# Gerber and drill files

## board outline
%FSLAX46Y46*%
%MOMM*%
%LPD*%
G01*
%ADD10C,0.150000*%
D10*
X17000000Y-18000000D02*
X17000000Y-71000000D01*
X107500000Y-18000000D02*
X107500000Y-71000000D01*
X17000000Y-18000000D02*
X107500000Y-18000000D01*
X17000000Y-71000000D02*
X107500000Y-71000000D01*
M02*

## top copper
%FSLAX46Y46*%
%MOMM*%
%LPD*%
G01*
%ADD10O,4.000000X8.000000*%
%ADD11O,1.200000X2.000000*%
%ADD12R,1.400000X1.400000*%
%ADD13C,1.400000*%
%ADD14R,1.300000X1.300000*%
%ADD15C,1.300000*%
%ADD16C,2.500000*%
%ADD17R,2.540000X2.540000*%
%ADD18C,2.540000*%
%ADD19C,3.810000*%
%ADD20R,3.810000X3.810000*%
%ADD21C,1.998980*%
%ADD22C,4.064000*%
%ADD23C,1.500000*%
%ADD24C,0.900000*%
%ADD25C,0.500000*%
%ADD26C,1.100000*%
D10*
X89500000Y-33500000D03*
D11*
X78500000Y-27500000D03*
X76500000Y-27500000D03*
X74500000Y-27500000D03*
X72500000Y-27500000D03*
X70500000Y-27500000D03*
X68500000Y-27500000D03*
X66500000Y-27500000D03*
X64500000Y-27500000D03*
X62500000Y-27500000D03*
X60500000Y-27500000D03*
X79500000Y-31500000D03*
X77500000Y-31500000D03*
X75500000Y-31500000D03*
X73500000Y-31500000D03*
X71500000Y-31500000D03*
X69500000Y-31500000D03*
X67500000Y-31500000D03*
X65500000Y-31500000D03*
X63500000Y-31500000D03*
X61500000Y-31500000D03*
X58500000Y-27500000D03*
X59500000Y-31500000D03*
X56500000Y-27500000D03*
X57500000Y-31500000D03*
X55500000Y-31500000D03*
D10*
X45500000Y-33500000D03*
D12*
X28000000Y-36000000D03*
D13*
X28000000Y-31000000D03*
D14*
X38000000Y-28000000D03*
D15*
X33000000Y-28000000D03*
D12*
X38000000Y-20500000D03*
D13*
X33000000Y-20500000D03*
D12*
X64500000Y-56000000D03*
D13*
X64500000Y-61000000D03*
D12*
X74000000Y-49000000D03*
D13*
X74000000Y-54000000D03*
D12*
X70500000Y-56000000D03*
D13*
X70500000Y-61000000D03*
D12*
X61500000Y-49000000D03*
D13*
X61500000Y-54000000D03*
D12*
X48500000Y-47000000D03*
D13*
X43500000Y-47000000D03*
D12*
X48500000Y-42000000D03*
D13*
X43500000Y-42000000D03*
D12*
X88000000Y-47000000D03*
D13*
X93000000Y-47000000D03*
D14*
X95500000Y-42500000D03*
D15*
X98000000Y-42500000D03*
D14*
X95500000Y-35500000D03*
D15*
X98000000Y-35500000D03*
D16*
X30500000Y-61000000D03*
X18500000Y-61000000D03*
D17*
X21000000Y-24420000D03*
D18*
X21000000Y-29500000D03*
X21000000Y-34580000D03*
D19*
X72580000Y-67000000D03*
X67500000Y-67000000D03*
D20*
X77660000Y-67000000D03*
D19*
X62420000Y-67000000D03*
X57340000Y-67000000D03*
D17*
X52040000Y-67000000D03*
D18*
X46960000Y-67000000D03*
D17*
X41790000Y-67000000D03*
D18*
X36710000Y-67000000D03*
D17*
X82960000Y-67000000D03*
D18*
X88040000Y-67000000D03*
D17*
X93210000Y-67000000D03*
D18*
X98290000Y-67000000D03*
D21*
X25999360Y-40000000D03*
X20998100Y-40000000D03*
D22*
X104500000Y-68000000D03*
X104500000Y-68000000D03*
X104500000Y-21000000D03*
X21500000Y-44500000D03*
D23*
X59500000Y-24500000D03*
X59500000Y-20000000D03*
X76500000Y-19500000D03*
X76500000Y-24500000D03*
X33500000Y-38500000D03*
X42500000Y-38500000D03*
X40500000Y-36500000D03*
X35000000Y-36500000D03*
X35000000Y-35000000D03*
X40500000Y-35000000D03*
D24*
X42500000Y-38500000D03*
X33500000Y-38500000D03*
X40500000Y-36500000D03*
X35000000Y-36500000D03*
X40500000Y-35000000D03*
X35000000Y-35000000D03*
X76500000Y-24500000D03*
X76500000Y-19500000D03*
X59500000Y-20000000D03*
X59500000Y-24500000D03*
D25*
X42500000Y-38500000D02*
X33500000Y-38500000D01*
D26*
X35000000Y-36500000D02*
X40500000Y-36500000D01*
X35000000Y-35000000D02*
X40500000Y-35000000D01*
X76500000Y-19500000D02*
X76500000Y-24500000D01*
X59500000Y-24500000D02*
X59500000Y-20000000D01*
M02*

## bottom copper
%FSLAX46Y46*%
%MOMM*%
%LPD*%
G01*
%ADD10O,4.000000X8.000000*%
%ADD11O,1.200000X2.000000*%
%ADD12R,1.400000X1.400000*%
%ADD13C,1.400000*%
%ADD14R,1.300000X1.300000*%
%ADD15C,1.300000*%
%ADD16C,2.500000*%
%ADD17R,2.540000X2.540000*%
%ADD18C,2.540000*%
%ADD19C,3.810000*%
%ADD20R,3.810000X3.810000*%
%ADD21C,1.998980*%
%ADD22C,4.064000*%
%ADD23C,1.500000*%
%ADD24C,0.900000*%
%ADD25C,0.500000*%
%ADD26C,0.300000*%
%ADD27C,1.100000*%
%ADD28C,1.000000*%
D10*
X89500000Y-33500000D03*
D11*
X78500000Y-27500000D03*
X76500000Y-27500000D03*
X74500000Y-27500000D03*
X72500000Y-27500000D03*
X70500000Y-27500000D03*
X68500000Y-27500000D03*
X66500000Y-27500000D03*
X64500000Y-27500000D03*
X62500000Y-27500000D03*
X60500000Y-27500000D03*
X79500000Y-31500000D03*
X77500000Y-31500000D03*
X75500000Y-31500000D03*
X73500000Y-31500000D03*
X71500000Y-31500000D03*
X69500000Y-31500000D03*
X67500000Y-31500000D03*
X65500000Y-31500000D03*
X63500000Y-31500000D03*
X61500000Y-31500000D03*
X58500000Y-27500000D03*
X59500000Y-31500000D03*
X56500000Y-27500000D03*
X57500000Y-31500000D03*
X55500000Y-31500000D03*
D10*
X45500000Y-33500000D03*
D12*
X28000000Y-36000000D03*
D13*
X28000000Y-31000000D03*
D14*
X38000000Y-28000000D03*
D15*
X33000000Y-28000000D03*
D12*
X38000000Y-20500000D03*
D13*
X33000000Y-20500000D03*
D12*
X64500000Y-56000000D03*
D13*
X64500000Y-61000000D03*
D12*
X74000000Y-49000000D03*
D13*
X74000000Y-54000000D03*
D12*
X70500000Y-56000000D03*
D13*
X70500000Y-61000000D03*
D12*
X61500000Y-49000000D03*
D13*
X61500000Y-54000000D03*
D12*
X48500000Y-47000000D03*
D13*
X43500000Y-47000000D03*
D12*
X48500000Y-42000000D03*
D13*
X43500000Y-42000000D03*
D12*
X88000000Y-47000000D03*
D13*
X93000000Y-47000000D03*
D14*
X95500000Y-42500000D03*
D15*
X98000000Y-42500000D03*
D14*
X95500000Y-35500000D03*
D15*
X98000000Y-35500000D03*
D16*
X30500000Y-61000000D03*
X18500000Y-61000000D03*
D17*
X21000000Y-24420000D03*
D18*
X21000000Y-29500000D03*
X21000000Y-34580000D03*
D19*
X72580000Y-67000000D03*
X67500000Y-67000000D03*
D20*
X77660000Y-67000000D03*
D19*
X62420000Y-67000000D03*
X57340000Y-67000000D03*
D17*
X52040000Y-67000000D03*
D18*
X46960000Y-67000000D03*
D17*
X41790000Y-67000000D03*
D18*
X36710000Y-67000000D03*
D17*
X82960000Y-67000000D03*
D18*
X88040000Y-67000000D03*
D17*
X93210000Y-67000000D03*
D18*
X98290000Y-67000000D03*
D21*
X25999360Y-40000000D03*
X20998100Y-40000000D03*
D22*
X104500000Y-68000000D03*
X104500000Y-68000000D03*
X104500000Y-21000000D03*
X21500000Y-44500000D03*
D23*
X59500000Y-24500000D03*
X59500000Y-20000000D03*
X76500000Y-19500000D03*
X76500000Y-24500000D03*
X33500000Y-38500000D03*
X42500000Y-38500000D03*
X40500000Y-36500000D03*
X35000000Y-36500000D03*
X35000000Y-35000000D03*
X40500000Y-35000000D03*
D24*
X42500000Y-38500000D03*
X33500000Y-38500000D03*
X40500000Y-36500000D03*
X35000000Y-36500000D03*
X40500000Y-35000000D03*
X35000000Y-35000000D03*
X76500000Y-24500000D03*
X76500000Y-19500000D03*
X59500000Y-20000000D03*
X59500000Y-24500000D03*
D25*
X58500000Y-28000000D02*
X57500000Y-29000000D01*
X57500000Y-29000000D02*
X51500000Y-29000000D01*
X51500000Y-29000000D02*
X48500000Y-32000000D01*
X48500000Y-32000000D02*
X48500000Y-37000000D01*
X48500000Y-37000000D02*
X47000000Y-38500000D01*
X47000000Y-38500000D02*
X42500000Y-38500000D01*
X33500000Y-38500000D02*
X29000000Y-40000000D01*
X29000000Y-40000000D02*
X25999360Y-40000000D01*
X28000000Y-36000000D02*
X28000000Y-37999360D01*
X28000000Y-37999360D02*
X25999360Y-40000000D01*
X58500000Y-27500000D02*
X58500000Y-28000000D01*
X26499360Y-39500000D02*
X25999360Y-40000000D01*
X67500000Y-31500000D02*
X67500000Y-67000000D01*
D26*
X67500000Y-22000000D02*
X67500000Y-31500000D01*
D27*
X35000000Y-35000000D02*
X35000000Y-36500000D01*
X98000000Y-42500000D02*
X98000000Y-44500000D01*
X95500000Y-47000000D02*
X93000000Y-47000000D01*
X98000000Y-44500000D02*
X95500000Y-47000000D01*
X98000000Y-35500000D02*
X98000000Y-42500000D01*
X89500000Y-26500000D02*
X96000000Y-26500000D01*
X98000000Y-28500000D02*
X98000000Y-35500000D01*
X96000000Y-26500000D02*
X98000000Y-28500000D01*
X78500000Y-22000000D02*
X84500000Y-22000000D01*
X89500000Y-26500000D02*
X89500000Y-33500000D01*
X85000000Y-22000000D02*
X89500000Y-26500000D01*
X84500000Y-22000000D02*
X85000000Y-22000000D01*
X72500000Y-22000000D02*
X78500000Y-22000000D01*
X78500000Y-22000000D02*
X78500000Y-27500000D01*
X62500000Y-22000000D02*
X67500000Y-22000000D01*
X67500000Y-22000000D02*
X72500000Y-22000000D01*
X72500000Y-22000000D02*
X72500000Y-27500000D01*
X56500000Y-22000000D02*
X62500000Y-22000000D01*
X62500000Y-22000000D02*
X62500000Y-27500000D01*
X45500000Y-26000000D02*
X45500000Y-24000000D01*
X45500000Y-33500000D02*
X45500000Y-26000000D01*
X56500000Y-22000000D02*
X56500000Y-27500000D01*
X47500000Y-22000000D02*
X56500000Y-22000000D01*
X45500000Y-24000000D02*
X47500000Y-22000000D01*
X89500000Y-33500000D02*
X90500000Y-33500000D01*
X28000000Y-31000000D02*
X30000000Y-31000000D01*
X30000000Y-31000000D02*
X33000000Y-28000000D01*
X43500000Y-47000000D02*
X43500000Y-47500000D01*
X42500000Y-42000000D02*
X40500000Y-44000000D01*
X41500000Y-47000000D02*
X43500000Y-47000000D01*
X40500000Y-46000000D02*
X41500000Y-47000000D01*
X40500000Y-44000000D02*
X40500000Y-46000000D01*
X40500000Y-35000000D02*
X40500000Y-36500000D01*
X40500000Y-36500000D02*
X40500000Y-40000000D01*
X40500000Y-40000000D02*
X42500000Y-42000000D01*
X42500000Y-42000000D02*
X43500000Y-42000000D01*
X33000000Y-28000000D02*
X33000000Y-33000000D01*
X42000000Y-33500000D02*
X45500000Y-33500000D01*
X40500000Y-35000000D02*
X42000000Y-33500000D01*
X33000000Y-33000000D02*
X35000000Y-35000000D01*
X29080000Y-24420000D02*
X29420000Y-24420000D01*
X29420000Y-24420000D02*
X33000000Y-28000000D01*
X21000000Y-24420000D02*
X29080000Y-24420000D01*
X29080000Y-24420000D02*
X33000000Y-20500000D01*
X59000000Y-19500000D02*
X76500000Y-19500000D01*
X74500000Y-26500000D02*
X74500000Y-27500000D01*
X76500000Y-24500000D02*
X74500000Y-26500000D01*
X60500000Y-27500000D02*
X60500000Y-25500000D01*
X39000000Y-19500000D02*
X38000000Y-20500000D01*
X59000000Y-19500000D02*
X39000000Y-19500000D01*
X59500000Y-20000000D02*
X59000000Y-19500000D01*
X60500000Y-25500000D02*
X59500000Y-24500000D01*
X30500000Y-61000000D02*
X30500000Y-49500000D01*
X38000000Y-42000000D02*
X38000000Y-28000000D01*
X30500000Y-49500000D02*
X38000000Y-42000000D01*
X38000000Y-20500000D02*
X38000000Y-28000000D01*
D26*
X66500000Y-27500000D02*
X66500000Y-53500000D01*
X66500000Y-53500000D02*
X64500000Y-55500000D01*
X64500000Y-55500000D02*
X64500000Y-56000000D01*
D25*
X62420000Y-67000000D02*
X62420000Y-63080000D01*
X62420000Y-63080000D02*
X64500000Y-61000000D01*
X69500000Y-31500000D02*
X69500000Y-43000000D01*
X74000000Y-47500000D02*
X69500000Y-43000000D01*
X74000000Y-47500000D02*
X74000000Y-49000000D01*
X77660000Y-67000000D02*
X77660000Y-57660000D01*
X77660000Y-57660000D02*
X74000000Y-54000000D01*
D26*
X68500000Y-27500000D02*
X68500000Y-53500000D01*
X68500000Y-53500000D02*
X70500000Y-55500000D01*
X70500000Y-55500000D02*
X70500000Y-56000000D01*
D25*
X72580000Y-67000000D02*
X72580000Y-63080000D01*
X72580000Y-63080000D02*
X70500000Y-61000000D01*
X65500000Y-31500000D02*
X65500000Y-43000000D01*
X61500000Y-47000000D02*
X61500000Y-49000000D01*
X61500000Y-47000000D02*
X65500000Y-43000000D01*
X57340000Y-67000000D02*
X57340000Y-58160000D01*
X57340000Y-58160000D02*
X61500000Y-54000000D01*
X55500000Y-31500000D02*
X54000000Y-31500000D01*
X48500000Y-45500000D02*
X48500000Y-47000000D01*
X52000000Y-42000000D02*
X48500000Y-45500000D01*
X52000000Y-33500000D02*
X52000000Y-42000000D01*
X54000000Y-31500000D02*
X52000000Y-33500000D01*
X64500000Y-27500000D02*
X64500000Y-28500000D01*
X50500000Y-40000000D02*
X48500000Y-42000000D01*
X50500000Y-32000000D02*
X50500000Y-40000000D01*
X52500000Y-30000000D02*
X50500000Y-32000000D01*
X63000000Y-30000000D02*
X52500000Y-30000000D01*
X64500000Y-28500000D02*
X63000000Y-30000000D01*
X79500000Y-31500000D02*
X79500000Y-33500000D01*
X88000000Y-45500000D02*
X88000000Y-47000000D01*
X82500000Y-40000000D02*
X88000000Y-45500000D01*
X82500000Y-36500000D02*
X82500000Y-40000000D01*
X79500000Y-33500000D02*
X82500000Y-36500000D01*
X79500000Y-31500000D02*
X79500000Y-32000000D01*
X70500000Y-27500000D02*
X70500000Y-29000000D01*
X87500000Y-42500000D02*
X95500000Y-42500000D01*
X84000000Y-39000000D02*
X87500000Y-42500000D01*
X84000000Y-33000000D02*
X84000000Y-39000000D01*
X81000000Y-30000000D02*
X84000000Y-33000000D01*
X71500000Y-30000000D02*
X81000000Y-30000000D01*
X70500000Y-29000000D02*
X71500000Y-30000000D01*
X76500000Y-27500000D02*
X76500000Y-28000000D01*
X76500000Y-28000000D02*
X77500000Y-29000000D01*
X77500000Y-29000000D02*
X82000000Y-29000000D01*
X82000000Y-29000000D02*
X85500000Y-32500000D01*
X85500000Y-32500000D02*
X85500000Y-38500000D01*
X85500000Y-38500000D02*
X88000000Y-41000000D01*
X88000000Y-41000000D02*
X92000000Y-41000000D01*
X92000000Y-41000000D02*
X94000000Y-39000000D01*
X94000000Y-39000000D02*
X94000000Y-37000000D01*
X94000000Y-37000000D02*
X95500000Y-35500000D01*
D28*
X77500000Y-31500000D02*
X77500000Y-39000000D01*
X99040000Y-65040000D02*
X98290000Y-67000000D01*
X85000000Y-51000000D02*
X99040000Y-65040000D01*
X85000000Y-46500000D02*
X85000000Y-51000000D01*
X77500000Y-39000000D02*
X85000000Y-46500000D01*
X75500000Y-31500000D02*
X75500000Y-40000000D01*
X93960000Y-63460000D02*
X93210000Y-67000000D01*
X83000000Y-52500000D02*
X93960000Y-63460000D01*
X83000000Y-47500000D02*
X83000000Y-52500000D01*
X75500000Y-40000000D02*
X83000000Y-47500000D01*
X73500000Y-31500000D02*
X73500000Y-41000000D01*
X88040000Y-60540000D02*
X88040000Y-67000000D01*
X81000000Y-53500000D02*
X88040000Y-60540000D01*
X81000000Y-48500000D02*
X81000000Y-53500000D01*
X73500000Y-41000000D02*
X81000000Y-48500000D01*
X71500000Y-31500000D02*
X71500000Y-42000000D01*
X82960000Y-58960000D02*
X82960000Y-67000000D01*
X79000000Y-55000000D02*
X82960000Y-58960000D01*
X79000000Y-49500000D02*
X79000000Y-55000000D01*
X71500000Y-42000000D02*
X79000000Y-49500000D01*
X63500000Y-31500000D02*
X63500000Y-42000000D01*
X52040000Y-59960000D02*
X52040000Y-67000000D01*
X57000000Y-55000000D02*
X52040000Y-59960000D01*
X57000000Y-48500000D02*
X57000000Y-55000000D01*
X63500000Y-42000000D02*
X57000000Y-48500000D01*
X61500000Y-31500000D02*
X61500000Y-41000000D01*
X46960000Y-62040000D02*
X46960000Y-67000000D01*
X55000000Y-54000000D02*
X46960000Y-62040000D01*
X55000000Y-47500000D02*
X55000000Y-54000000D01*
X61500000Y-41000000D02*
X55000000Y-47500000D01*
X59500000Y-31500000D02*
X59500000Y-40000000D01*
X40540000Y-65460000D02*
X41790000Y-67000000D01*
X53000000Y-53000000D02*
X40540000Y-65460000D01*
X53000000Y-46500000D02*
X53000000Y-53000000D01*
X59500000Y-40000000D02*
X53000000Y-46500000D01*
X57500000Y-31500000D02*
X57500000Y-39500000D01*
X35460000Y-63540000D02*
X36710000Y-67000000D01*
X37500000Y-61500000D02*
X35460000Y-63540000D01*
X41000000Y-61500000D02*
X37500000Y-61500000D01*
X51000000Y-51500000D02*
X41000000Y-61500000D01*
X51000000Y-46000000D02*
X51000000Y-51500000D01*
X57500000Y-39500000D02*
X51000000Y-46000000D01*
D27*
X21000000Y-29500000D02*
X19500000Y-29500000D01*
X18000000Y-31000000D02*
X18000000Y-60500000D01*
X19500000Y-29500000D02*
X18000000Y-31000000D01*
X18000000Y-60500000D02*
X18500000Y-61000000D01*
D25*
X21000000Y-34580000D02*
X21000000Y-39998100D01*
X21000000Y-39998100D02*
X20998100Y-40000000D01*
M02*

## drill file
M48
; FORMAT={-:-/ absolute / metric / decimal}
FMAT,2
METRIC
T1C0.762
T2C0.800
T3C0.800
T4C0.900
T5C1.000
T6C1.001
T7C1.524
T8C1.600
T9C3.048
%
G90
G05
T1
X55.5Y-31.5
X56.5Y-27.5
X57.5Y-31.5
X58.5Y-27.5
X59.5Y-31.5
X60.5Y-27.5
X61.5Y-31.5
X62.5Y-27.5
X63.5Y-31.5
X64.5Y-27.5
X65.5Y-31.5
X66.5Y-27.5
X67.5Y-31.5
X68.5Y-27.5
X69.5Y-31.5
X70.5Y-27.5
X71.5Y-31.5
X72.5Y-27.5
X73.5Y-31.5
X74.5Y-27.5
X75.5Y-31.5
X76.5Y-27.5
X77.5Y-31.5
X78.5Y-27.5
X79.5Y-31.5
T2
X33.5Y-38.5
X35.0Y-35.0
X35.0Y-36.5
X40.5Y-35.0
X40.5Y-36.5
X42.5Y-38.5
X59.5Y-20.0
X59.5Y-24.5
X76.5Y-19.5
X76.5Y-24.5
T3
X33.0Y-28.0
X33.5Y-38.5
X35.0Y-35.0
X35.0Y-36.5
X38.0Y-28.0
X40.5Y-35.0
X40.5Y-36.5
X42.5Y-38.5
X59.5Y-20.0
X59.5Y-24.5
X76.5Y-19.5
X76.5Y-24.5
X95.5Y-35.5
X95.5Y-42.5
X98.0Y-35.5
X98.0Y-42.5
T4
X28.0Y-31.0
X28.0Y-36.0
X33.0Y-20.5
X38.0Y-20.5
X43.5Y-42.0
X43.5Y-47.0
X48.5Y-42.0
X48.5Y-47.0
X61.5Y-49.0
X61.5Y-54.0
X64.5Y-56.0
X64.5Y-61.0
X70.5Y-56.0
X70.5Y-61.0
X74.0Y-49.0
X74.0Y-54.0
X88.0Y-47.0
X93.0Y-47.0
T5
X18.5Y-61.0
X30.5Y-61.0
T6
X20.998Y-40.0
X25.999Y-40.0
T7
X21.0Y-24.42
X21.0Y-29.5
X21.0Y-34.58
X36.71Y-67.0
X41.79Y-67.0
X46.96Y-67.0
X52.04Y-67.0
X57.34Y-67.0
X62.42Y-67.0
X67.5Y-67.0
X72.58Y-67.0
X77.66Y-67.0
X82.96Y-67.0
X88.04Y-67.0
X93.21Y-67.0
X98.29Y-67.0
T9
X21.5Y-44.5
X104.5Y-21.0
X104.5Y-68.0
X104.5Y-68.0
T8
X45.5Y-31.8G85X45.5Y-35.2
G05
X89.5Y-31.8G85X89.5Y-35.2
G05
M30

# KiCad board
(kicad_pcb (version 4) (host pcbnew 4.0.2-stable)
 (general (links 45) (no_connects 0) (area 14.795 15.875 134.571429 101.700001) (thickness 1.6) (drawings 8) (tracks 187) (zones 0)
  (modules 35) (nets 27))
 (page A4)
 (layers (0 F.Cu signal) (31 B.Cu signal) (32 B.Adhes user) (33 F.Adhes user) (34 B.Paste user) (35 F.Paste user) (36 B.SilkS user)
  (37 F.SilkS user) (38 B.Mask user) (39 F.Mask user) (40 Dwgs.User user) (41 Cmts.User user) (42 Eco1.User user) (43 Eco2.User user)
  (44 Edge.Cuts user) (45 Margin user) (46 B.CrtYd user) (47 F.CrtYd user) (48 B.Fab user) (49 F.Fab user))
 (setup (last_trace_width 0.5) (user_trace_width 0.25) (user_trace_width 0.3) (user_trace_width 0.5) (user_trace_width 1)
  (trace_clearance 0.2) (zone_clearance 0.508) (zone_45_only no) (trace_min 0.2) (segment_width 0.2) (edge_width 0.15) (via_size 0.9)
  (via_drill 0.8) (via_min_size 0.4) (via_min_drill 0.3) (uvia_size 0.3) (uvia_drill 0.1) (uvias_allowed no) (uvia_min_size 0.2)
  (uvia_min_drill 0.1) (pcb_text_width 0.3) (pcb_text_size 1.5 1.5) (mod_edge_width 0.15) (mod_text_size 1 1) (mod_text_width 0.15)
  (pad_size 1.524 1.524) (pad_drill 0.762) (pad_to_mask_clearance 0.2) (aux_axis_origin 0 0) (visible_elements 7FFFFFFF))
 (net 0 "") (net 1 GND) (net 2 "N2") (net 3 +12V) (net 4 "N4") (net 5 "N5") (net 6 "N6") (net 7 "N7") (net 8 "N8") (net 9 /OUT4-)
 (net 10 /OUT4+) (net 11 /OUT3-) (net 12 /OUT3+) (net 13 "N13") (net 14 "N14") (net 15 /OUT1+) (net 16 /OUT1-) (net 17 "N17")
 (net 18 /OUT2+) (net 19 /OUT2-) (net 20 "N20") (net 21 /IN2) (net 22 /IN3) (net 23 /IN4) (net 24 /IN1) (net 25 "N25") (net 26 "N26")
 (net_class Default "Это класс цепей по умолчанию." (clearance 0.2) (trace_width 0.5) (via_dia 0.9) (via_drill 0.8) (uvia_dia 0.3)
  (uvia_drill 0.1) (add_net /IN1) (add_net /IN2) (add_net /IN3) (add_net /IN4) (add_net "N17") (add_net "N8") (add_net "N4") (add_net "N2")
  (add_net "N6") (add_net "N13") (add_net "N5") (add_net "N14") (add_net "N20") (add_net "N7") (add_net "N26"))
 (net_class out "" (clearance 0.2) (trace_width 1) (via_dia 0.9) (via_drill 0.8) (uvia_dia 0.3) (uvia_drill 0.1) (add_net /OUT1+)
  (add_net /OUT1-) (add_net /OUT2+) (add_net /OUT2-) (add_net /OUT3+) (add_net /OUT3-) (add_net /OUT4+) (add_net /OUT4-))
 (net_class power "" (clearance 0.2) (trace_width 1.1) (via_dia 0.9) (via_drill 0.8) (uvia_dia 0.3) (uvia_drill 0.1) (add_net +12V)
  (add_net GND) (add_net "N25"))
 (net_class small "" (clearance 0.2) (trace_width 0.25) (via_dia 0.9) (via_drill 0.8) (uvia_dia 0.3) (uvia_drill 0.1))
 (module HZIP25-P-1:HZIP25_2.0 (layer F.Cu) (at 55.5 31.5)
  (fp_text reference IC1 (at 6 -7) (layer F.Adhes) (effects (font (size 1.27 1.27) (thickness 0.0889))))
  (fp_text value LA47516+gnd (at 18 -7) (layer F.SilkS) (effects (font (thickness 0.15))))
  (pad GND2 thru_hole oval (at 34 2) (size 4 8) (drill oval 1.6 5) (layers *.Cu F.Paste F.SilkS F.Mask) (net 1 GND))
  (pad 24 thru_hole oval (at 23 -4) (size 1.2 2) (drill 0.762) (layers *.Cu F.Paste F.SilkS F.Mask) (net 1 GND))
  (pad 22 thru_hole oval (at 21 -4) (size 1.2 2) (drill 0.762) (layers *.Cu F.Paste F.SilkS F.Mask) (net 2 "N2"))
  (pad 20 thru_hole oval (at 19 -4) (size 1.2 2) (drill 0.762) (layers *.Cu F.Paste F.SilkS F.Mask) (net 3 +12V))
  (pad 18 thru_hole oval (at 17 -4) (size 1.2 2) (drill 0.762) (layers *.Cu F.Paste F.SilkS F.Mask) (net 1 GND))
  (pad 16 thru_hole oval (at 15 -4) (size 1.2 2) (drill 0.762) (layers *.Cu F.Paste F.SilkS F.Mask) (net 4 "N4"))
  (pad 14 thru_hole oval (at 13 -4) (size 1.2 2) (drill 0.762) (layers *.Cu F.Paste F.SilkS F.Mask) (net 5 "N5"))
  (pad 12 thru_hole oval (at 11 -4) (size 1.2 2) (drill 0.762) (layers *.Cu F.Paste F.SilkS F.Mask) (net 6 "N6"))
  (pad 10 thru_hole oval (at 9 -4) (size 1.2 2) (drill 0.762) (layers *.Cu F.Paste F.SilkS F.Mask) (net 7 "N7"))
  (pad 8 thru_hole oval (at 7 -4) (size 1.2 2) (drill 0.762) (layers *.Cu F.Paste F.SilkS F.Mask) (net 1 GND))
  (pad 6 thru_hole oval (at 5 -4) (size 1.2 2) (drill 0.762) (layers *.Cu F.Paste F.SilkS F.Mask) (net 3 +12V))
  (pad 25 thru_hole oval (at 24 0) (size 1.2 2) (drill 0.762) (layers *.Cu F.Paste F.SilkS F.Mask) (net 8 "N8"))
  (pad 23 thru_hole oval (at 22 0) (size 1.2 2) (drill 0.762) (layers *.Cu F.Paste F.SilkS F.Mask) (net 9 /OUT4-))
  (pad 21 thru_hole oval (at 20 0) (size 1.2 2) (drill 0.762) (layers *.Cu F.Paste F.SilkS F.Mask) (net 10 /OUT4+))
  (pad 19 thru_hole oval (at 18 0) (size 1.2 2) (drill 0.762) (layers *.Cu F.Paste F.SilkS F.Mask) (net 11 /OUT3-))
  (pad 17 thru_hole oval (at 16 0) (size 1.2 2) (drill 0.762) (layers *.Cu F.Paste F.SilkS F.Mask) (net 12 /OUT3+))
  (pad 15 thru_hole oval (at 14 0) (size 1.2 2) (drill 0.762) (layers *.Cu F.Paste F.SilkS F.Mask) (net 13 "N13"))
  (pad 13 thru_hole oval (at 12 0) (size 1.2 2) (drill 0.762) (layers *.Cu F.Paste F.SilkS F.Mask) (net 1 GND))
  (pad 11 thru_hole oval (at 10 0) (size 1.2 2) (drill 0.762) (layers *.Cu F.Paste F.SilkS F.Mask) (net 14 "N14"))
  (pad 9 thru_hole oval (at 8 0) (size 1.2 2) (drill 0.762) (layers *.Cu F.Paste F.SilkS F.Mask) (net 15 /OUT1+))
  (pad 7 thru_hole oval (at 6 0) (size 1.2 2) (drill 0.762) (layers *.Cu F.Paste F.SilkS F.Mask) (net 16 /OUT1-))
  (pad 4 thru_hole oval (at 3 -4) (size 1.2 2) (drill 0.762) (layers *.Cu F.Paste F.SilkS F.Mask) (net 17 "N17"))
  (pad 5 thru_hole oval (at 4 0) (size 1.2 2) (drill 0.762) (layers *.Cu F.Paste F.SilkS F.Mask) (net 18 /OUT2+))
  (pad 2 thru_hole oval (at 1 -4) (size 1.2 2) (drill 0.762) (layers *.Cu F.Paste F.SilkS F.Mask) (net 1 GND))
  (pad 3 thru_hole oval (at 2 0) (size 1.2 2) (drill 0.762) (layers *.Cu F.Paste F.SilkS F.Mask) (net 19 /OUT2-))
  (pad 1 thru_hole oval (at 0 0) (size 1.2 2) (drill 0.762) (layers *.Cu F.Paste F.SilkS F.Mask) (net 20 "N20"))
  (pad GND1 thru_hole oval (at -10 2) (size 4 8) (drill oval 1.6 5) (layers *.Cu *.Mask F.SilkS) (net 1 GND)))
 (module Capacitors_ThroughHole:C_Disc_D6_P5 (layer F.Cu) (at 28 36 90)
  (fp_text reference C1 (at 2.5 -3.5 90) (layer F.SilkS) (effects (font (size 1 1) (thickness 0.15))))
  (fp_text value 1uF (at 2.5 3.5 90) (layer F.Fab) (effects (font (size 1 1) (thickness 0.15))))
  (pad 1 thru_hole rect (at 0 0 90) (size 1.4 1.4) (drill 0.9) (layers *.Cu *.Mask F.SilkS) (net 17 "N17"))
  (pad 2 thru_hole circle (at 5 0 90) (size 1.4 1.4) (drill 0.9) (layers *.Cu *.Mask F.SilkS) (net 1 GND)))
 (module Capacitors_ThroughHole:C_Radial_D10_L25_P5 (layer F.Cu) (at 38 28 180)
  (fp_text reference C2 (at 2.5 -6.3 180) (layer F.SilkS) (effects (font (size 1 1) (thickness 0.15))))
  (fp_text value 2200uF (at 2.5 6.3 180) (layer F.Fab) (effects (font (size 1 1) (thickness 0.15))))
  (pad 1 thru_hole rect (at 0 0 180) (size 1.3 1.3) (drill 0.8) (layers *.Cu *.Mask F.SilkS) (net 3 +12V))
  (pad 2 thru_hole circle (at 5 0 180) (size 1.3 1.3) (drill 0.8) (layers *.Cu *.Mask F.SilkS) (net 1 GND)))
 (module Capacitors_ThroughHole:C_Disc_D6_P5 (layer F.Cu) (at 38 20.5 180)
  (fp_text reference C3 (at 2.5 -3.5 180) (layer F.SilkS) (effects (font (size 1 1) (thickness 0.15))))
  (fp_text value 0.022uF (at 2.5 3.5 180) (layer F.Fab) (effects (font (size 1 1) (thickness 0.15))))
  (pad 1 thru_hole rect (at 0 0 180) (size 1.4 1.4) (drill 0.9) (layers *.Cu *.Mask F.SilkS) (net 3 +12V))
  (pad 2 thru_hole circle (at 5 0 180) (size 1.4 1.4) (drill 0.9) (layers *.Cu *.Mask F.SilkS) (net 1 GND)))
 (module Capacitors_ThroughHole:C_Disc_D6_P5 (layer F.Cu) (at 64.5 56 270)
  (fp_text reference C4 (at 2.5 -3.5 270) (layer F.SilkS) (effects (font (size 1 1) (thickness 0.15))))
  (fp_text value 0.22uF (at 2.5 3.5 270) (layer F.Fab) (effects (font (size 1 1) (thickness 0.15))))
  (pad 1 thru_hole rect (at 0 0 270) (size 1.4 1.4) (drill 0.9) (layers *.Cu *.Mask F.SilkS) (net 6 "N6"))
  (pad 2 thru_hole circle (at 5 0 270) (size 1.4 1.4) (drill 0.9) (layers *.Cu *.Mask F.SilkS) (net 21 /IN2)))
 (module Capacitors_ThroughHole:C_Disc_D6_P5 (layer F.Cu) (at 74 49 270)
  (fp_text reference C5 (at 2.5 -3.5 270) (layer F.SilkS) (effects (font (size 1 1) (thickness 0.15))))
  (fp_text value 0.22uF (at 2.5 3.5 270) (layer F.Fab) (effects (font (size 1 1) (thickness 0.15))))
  (pad 1 thru_hole rect (at 0 0 270) (size 1.4 1.4) (drill 0.9) (layers *.Cu *.Mask F.SilkS) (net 13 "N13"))
  (pad 2 thru_hole circle (at 5 0 270) (size 1.4 1.4) (drill 0.9) (layers *.Cu *.Mask F.SilkS) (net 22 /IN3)))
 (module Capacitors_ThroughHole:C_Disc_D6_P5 (layer F.Cu) (at 70.5 56 270)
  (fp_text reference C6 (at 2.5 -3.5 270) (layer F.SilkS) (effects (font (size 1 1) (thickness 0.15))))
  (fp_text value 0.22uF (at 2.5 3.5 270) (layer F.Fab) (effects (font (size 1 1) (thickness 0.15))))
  (pad 1 thru_hole rect (at 0 0 270) (size 1.4 1.4) (drill 0.9) (layers *.Cu *.Mask F.SilkS) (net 5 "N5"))
  (pad 2 thru_hole circle (at 5 0 270) (size 1.4 1.4) (drill 0.9) (layers *.Cu *.Mask F.SilkS) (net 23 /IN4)))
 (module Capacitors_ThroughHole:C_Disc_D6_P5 (layer F.Cu) (at 61.5 49 270)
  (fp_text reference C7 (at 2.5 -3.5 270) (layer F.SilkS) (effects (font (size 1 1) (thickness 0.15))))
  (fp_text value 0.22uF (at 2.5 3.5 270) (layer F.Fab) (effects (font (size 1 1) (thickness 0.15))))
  (pad 1 thru_hole rect (at 0 0 270) (size 1.4 1.4) (drill 0.9) (layers *.Cu *.Mask F.SilkS) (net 14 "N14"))
  (pad 2 thru_hole circle (at 5 0 270) (size 1.4 1.4) (drill 0.9) (layers *.Cu *.Mask F.SilkS) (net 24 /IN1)))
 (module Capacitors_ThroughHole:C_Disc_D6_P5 (layer F.Cu) (at 48.5 47 180)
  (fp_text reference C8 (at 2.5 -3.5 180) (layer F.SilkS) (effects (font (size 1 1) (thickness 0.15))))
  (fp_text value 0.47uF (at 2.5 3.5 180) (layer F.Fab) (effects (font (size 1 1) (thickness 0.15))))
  (pad 1 thru_hole rect (at 0 0 180) (size 1.4 1.4) (drill 0.9) (layers *.Cu *.Mask F.SilkS) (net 20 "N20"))
  (pad 2 thru_hole circle (at 5 0 180) (size 1.4 1.4) (drill 0.9) (layers *.Cu *.Mask F.SilkS) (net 1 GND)))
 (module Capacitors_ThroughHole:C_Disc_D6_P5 (layer F.Cu) (at 48.5 42 180)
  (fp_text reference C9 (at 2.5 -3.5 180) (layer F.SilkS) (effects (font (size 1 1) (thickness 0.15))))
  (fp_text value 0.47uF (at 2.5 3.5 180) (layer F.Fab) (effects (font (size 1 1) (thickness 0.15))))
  (pad 1 thru_hole rect (at 0 0 180) (size 1.4 1.4) (drill 0.9) (layers *.Cu *.Mask F.SilkS) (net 7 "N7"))
  (pad 2 thru_hole circle (at 5 0 180) (size 1.4 1.4) (drill 0.9) (layers *.Cu *.Mask F.SilkS) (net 1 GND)))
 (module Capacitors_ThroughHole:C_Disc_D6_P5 (layer F.Cu) (at 88 47)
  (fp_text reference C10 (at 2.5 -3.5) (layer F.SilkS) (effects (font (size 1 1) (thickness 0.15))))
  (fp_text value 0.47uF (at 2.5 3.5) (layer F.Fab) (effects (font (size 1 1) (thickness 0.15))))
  (pad 1 thru_hole rect (at 0 0) (size 1.4 1.4) (drill 0.9) (layers *.Cu *.Mask F.SilkS) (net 8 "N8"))
  (pad 2 thru_hole circle (at 5 0) (size 1.4 1.4) (drill 0.9) (layers *.Cu *.Mask F.SilkS) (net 1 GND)))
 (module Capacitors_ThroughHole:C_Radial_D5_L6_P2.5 (layer F.Cu) (at 95.5 42.5)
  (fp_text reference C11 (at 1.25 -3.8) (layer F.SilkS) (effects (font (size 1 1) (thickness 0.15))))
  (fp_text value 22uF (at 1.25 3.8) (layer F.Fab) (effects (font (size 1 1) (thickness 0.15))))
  (pad 1 thru_hole rect (at 0 0) (size 1.3 1.3) (drill 0.8) (layers *.Cu *.Mask F.SilkS) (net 4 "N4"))
  (pad 2 thru_hole circle (at 2.5 0) (size 1.3 1.3) (drill 0.8) (layers *.Cu *.Mask F.SilkS) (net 1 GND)))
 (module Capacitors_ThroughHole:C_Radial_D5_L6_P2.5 (layer F.Cu) (at 95.5 35.5)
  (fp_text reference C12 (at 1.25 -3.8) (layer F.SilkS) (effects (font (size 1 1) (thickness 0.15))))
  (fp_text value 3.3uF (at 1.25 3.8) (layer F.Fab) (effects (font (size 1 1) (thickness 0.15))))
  (pad 1 thru_hole rect (at 0 0) (size 1.3 1.3) (drill 0.8) (layers *.Cu *.Mask F.SilkS) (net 2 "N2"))
  (pad 2 thru_hole circle (at 2.5 0) (size 1.3 1.3) (drill 0.8) (layers *.Cu *.Mask F.SilkS) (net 1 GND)))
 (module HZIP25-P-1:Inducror (layer F.Cu) (at 24.5 61 90)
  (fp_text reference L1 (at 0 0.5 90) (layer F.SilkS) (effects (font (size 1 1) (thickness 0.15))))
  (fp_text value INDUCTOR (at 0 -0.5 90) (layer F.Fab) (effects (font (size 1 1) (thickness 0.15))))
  (pad 2 thru_hole circle (at 0 6 90) (size 2.5 2.5) (drill 1) (layers *.Cu *.Mask F.SilkS) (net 3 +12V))
  (pad 1 thru_hole circle (at 0 -6 90) (size 2.5 2.5) (drill 1) (layers *.Cu *.Mask F.SilkS) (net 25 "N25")))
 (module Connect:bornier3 (layer F.Cu) (at 21 29.5 270)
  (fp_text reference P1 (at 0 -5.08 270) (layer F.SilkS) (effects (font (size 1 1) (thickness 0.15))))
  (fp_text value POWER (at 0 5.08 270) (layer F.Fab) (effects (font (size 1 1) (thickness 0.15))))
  (pad 1 thru_hole rect (at -5.08 0 270) (size 2.54 2.54) (drill 1.524) (layers *.Cu *.Mask F.SilkS) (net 1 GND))
  (pad 2 thru_hole circle (at 0 0 270) (size 2.54 2.54) (drill 1.524) (layers *.Cu *.Mask F.SilkS) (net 25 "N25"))
  (pad 3 thru_hole circle (at 5.08 0 270) (size 2.54 2.54) (drill 1.524) (layers *.Cu *.Mask F.SilkS) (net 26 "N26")))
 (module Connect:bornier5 (layer F.Cu) (at 67.5 67 180)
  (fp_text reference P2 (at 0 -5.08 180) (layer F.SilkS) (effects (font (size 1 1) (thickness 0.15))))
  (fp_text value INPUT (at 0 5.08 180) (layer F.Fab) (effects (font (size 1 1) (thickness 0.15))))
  (pad 2 thru_hole circle (at -5.08 0 180) (size 3.81 3.81) (drill 1.524) (layers *.Cu *.Mask F.SilkS) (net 23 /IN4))
  (pad 3 thru_hole circle (at 0 0 180) (size 3.81 3.81) (drill 1.524) (layers *.Cu *.Mask F.SilkS) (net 1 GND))
  (pad 1 thru_hole rect (at -10.16 0 180) (size 3.81 3.81) (drill 1.524) (layers *.Cu *.Mask F.SilkS) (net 22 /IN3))
  (pad 4 thru_hole circle (at 5.08 0 180) (size 3.81 3.81) (drill 1.524) (layers *.Cu *.Mask F.SilkS) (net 21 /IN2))
  (pad 5 thru_hole circle (at 10.16 0 180) (size 3.81 3.81) (drill 1.524) (layers *.Cu *.Mask F.SilkS) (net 24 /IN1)))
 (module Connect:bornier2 (layer F.Cu) (at 49.5 67 180)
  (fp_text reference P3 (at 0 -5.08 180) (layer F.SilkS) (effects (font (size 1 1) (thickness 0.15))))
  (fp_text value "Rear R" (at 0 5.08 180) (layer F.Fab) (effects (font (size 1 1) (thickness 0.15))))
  (pad 1 thru_hole rect (at -2.54 0 180) (size 2.54 2.54) (drill 1.524) (layers *.Cu *.Mask F.SilkS) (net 15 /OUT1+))
  (pad 2 thru_hole circle (at 2.54 0 180) (size 2.54 2.54) (drill 1.524) (layers *.Cu *.Mask F.SilkS) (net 16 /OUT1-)))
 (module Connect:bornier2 (layer F.Cu) (at 39.25 67 180)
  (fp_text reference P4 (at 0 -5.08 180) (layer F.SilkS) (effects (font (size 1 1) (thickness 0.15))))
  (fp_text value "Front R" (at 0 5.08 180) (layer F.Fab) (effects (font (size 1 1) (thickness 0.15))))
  (pad 1 thru_hole rect (at -2.54 0 180) (size 2.54 2.54) (drill 1.524) (layers *.Cu *.Mask F.SilkS) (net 18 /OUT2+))
  (pad 2 thru_hole circle (at 2.54 0 180) (size 2.54 2.54) (drill 1.524) (layers *.Cu *.Mask F.SilkS) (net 19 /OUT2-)))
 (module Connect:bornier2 (layer F.Cu) (at 85.5 67)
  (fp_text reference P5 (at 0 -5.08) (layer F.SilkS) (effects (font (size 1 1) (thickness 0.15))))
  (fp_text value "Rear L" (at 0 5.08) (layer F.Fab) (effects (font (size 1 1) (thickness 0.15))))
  (pad 1 thru_hole rect (at -2.54 0) (size 2.54 2.54) (drill 1.524) (layers *.Cu *.Mask F.SilkS) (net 12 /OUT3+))
  (pad 2 thru_hole circle (at 2.54 0) (size 2.54 2.54) (drill 1.524) (layers *.Cu *.Mask F.SilkS) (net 11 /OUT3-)))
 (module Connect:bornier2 (layer F.Cu) (at 95.75 67)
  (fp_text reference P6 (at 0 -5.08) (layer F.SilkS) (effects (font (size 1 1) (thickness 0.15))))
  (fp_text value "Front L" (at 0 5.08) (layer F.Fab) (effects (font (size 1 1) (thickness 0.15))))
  (pad 1 thru_hole rect (at -2.54 0) (size 2.54 2.54) (drill 1.524) (layers *.Cu *.Mask F.SilkS) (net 10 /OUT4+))
  (pad 2 thru_hole circle (at 2.54 0) (size 2.54 2.54) (drill 1.524) (layers *.Cu *.Mask F.SilkS) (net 9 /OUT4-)))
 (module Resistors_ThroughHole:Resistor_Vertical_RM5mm (layer F.Cu) (at 23.5 40 180)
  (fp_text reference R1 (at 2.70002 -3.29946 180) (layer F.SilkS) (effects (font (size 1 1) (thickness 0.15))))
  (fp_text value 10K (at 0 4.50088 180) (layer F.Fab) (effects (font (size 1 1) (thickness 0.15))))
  (pad 1 thru_hole circle (at -2.49936 0 180) (size 1.99898 1.99898) (drill 1.00076) (layers *.Cu *.SilkS *.Mask) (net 17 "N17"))
  (pad 2 thru_hole circle (at 2.5019 0 180) (size 1.99898 1.99898) (drill 1.00076) (layers *.Cu *.SilkS *.Mask) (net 26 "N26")))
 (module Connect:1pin (layer F.Cu) (at 104.5 68)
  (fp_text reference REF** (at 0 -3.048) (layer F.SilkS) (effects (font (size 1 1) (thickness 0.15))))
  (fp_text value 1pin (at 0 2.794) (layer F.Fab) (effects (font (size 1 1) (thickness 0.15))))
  (pad 1 thru_hole circle (at 0 0) (size 4.064 4.064) (drill 3.048) (layers *.Cu *.Mask F.SilkS)))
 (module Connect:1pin (layer F.Cu) (at 104.5 68)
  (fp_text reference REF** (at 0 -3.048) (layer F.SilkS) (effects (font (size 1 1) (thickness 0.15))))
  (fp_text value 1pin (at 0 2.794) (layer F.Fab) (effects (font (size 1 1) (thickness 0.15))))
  (pad 1 thru_hole circle (at 0 0) (size 4.064 4.064) (drill 3.048) (layers *.Cu *.Mask F.SilkS)))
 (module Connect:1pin (layer F.Cu) (at 104.5 21)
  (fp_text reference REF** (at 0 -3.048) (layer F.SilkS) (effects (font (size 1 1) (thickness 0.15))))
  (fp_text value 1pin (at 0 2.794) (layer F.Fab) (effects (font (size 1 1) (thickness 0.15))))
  (pad 1 thru_hole circle (at 0 0) (size 4.064 4.064) (drill 3.048) (layers *.Cu *.Mask F.SilkS)))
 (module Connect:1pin (layer F.Cu) (at 21.5 44.5)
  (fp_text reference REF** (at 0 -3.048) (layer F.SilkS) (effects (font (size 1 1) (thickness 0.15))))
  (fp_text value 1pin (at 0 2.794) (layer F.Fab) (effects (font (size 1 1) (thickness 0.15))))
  (pad 1 thru_hole circle (at 0 0) (size 4.064 4.064) (drill 3.048) (layers *.Cu *.Mask F.SilkS)))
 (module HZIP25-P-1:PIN (layer F.Cu) (at 59.5 24.5)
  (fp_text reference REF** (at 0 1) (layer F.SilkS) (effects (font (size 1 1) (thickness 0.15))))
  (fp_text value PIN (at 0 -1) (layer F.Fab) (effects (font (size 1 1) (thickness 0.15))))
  (pad 1 thru_hole circle (at 0 0) (size 1.5 1.5) (drill 0.8) (layers *.Cu *.Mask F.SilkS)))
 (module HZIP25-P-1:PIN (layer F.Cu) (at 59.5 20)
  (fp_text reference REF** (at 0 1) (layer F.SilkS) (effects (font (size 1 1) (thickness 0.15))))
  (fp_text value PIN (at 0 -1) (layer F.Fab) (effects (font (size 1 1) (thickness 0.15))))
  (pad 1 thru_hole circle (at 0 0) (size 1.5 1.5) (drill 0.8) (layers *.Cu *.Mask F.SilkS)))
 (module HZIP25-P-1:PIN (layer F.Cu) (at 76.5 19.5)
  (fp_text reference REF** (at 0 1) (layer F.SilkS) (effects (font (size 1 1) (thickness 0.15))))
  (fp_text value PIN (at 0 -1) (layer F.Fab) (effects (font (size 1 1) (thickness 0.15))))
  (pad 1 thru_hole circle (at 0 0) (size 1.5 1.5) (drill 0.8) (layers *.Cu *.Mask F.SilkS)))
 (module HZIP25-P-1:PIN (layer F.Cu) (at 76.5 24.5)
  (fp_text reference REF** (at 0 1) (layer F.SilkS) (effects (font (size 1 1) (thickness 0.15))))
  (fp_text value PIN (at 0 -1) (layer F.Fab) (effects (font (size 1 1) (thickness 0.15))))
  (pad 1 thru_hole circle (at 0 0) (size 1.5 1.5) (drill 0.8) (layers *.Cu *.Mask F.SilkS)))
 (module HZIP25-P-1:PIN (layer F.Cu) (at 33.5 38.5)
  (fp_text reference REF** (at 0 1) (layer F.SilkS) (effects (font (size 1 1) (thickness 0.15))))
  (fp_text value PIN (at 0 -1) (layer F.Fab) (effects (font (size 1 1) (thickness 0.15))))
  (pad 1 thru_hole circle (at 0 0) (size 1.5 1.5) (drill 0.8) (layers *.Cu *.Mask F.SilkS)))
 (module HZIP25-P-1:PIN (layer F.Cu) (at 42.5 38.5)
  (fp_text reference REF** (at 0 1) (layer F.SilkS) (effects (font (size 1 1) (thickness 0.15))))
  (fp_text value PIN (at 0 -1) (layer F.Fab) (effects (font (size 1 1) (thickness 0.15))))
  (pad 1 thru_hole circle (at 0 0) (size 1.5 1.5) (drill 0.8) (layers *.Cu *.Mask F.SilkS)))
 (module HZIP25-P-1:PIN (layer F.Cu) (at 40.5 36.5)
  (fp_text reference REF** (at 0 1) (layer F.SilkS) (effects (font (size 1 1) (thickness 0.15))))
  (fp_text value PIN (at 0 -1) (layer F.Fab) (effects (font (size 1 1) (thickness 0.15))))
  (pad 1 thru_hole circle (at 0 0) (size 1.5 1.5) (drill 0.8) (layers *.Cu *.Mask F.SilkS)))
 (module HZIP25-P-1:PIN (layer F.Cu) (at 35 36.5)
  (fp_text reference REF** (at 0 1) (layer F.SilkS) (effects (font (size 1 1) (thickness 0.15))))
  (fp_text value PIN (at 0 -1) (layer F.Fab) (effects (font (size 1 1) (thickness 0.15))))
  (pad 1 thru_hole circle (at 0 0) (size 1.5 1.5) (drill 0.8) (layers *.Cu *.Mask F.SilkS)))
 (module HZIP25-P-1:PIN (layer F.Cu) (at 35 35)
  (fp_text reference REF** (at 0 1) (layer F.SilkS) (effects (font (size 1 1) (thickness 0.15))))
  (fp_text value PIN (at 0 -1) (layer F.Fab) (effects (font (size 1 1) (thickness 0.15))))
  (pad 1 thru_hole circle (at 0 0) (size 1.5 1.5) (drill 0.8) (layers *.Cu *.Mask F.SilkS)))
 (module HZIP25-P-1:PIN (layer F.Cu) (at 40.5 35)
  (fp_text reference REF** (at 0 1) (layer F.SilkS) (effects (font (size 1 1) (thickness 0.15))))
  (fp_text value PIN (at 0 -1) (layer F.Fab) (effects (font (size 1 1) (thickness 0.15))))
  (pad 1 thru_hole circle (at 0 0) (size 1.5 1.5) (drill 0.8) (layers *.Cu *.Mask F.SilkS)))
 (gr_line (start 17 18) (end 17 71) (angle 90) (layer Edge.Cuts) (width 0.15))
 (gr_line (start 107.5 18) (end 107.5 71) (angle 90) (layer Edge.Cuts) (width 0.15))
 (gr_line (start 17 18) (end 107.5 18) (angle 90) (layer Edge.Cuts) (width 0.15))
 (gr_line (start 17 71) (end 107.5 71) (angle 90) (layer Edge.Cuts) (width 0.15))
 (segment (start 58.5 28) (end 57.5 29) (width 0.5) (layer B.Cu) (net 17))
 (segment (start 57.5 29) (end 51.5 29) (width 0.5) (layer B.Cu) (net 17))
 (segment (start 51.5 29) (end 48.5 32) (width 0.5) (layer B.Cu) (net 17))
 (segment (start 48.5 32) (end 48.5 37) (width 0.5) (layer B.Cu) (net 17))
 (segment (start 48.5 37) (end 47 38.5) (width 0.5) (layer B.Cu) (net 17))
 (segment (start 47 38.5) (end 42.5 38.5) (width 0.5) (layer B.Cu) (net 17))
 (via (at 42.5 38.5) (size 0.9) (drill 0.8) (layers F.Cu B.Cu) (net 17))
 (segment (start 42.5 38.5) (end 33.5 38.5) (width 0.5) (layer F.Cu) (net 17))
 (via (at 33.5 38.5) (size 0.9) (drill 0.8) (layers F.Cu B.Cu) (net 17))
 (segment (start 33.5 38.5) (end 29 40) (width 0.5) (layer B.Cu) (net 17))
 (segment (start 29 40) (end 25.99936 40) (width 0.5) (layer B.Cu) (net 17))
 (segment (start 28 36) (end 28 37.99936) (width 0.5) (layer B.Cu) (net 17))
 (segment (start 28 37.99936) (end 25.99936 40) (width 0.5) (layer B.Cu) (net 17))
 (segment (start 58.5 27.5) (end 58.5 28) (width 0.5) (layer B.Cu) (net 17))
 (segment (start 26.49936 39.5) (end 25.99936 40) (width 0.5) (layer B.Cu) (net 17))
 (segment (start 67.5 31.5) (end 67.5 67) (width 0.5) (layer B.Cu) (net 1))
 (segment (start 67.5 22) (end 67.5 31.5) (width 0.3) (layer B.Cu) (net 1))
 (segment (start 35 35) (end 35 36.5) (width 1.1) (layer B.Cu) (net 1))
 (via (at 40.5 36.5) (size 0.9) (drill 0.8) (layers F.Cu B.Cu) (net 1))
 (segment (start 35 36.5) (end 40.5 36.5) (width 1.1) (layer F.Cu) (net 1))
 (via (at 35 36.5) (size 0.9) (drill 0.8) (layers F.Cu B.Cu) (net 1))
 (segment (start 98 42.5) (end 98 44.5) (width 1.1) (layer B.Cu) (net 1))
 (segment (start 95.5 47) (end 93 47) (width 1.1) (layer B.Cu) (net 1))
 (segment (start 98 44.5) (end 95.5 47) (width 1.1) (layer B.Cu) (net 1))
 (segment (start 98 35.5) (end 98 42.5) (width 1.1) (layer B.Cu) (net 1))
 (segment (start 89.5 26.5) (end 96 26.5) (width 1.1) (layer B.Cu) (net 1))
 (segment (start 98 28.5) (end 98 35.5) (width 1.1) (layer B.Cu) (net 1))
 (segment (start 96 26.5) (end 98 28.5) (width 1.1) (layer B.Cu) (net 1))
 (segment (start 78.5 22) (end 84.5 22) (width 1.1) (layer B.Cu) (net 1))
 (segment (start 89.5 26.5) (end 89.5 33.5) (width 1.1) (layer B.Cu) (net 1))
 (segment (start 85 22) (end 89.5 26.5) (width 1.1) (layer B.Cu) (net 1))
 (segment (start 84.5 22) (end 85 22) (width 1.1) (layer B.Cu) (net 1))
 (segment (start 72.5 22) (end 78.5 22) (width 1.1) (layer B.Cu) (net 1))
 (segment (start 78.5 22) (end 78.5 27.5) (width 1.1) (layer B.Cu) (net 1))
 (segment (start 62.5 22) (end 67.5 22) (width 1.1) (layer B.Cu) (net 1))
 (segment (start 67.5 22) (end 72.5 22) (width 1.1) (layer B.Cu) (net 1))
 (segment (start 72.5 22) (end 72.5 27.5) (width 1.1) (layer B.Cu) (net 1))
 (segment (start 56.5 22) (end 62.5 22) (width 1.1) (layer B.Cu) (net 1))
 (segment (start 62.5 22) (end 62.5 27.5) (width 1.1) (layer B.Cu) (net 1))
 (segment (start 45.5 26) (end 45.5 24) (width 1.1) (layer B.Cu) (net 1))
 (segment (start 45.5 33.5) (end 45.5 26) (width 1.1) (layer B.Cu) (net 1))
 (segment (start 56.5 22) (end 56.5 27.5) (width 1.1) (layer B.Cu) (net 1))
 (segment (start 47.5 22) (end 56.5 22) (width 1.1) (layer B.Cu) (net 1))
 (segment (start 45.5 24) (end 47.5 22) (width 1.1) (layer B.Cu) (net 1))
 (segment (start 89.5 33.5) (end 90.5 33.5) (width 1.1) (layer B.Cu) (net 1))
 (segment (start 28 31) (end 30 31) (width 1.1) (layer B.Cu) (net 1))
 (segment (start 30 31) (end 33 28) (width 1.1) (layer B.Cu) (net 1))
 (segment (start 43.5 47) (end 43.5 47.5) (width 1.1) (layer B.Cu) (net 1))
 (segment (start 42.5 42) (end 40.5 44) (width 1.1) (layer B.Cu) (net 1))
 (segment (start 41.5 47) (end 43.5 47) (width 1.1) (layer B.Cu) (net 1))
 (segment (start 40.5 46) (end 41.5 47) (width 1.1) (layer B.Cu) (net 1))
 (segment (start 40.5 44) (end 40.5 46) (width 1.1) (layer B.Cu) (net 1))
 (segment (start 40.5 35) (end 40.5 36.5) (width 1.1) (layer B.Cu) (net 1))
 (segment (start 40.5 36.5) (end 40.5 40) (width 1.1) (layer B.Cu) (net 1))
 (segment (start 40.5 40) (end 42.5 42) (width 1.1) (layer B.Cu) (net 1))
 (segment (start 42.5 42) (end 43.5 42) (width 1.1) (layer B.Cu) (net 1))
 (segment (start 33 28) (end 33 33) (width 1.1) (layer B.Cu) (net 1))
 (segment (start 42 33.5) (end 45.5 33.5) (width 1.1) (layer B.Cu) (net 1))
 (segment (start 40.5 35) (end 42 33.5) (width 1.1) (layer B.Cu) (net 1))
 (via (at 40.5 35) (size 0.9) (drill 0.8) (layers F.Cu B.Cu) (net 1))
 (segment (start 35 35) (end 40.5 35) (width 1.1) (layer F.Cu) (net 1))
 (via (at 35 35) (size 0.9) (drill 0.8) (layers F.Cu B.Cu) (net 1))
 (segment (start 33 33) (end 35 35) (width 1.1) (layer B.Cu) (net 1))
 (segment (start 29.08 24.42) (end 29.42 24.42) (width 1.1) (layer B.Cu) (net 1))
 (segment (start 29.42 24.42) (end 33 28) (width 1.1) (layer B.Cu) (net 1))
 (segment (start 21 24.42) (end 29.08 24.42) (width 1.1) (layer B.Cu) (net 1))
 (segment (start 29.08 24.42) (end 33 20.5) (width 1.1) (layer B.Cu) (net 1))
 (segment (start 59 19.5) (end 76.5 19.5) (width 1.1) (layer B.Cu) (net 3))
 (segment (start 74.5 26.5) (end 74.5 27.5) (width 1.1) (layer B.Cu) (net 3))
 (segment (start 76.5 24.5) (end 74.5 26.5) (width 1.1) (layer B.Cu) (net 3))
 (via (at 76.5 24.5) (size 0.9) (drill 0.8) (layers F.Cu B.Cu) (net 3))
 (segment (start 76.5 19.5) (end 76.5 24.5) (width 1.1) (layer F.Cu) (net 3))
 (via (at 76.5 19.5) (size 0.9) (drill 0.8) (layers F.Cu B.Cu) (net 3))
 (segment (start 60.5 27.5) (end 60.5 25.5) (width 1.1) (layer B.Cu) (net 3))
 (segment (start 39 19.5) (end 38 20.5) (width 1.1) (layer B.Cu) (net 3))
 (segment (start 59 19.5) (end 39 19.5) (width 1.1) (layer B.Cu) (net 3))
 (segment (start 59.5 20) (end 59 19.5) (width 1.1) (layer B.Cu) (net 3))
 (via (at 59.5 20) (size 0.9) (drill 0.8) (layers F.Cu B.Cu) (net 3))
 (segment (start 59.5 24.5) (end 59.5 20) (width 1.1) (layer F.Cu) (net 3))
 (via (at 59.5 24.5) (size 0.9) (drill 0.8) (layers F.Cu B.Cu) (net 3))
 (segment (start 60.5 25.5) (end 59.5 24.5) (width 1.1) (layer B.Cu) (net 3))
 (segment (start 30.5 61) (end 30.5 49.5) (width 1.1) (layer B.Cu) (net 3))
 (segment (start 38 42) (end 38 28) (width 1.1) (layer B.Cu) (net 3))
 (segment (start 30.5 49.5) (end 38 42) (width 1.1) (layer B.Cu) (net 3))
 (segment (start 38 20.5) (end 38 28) (width 1.1) (layer B.Cu) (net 3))
 (segment (start 66.5 27.5) (end 66.5 53.5) (width 0.3) (layer B.Cu) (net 6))
 (segment (start 66.5 53.5) (end 64.5 55.5) (width 0.3) (layer B.Cu) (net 6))
 (segment (start 64.5 55.5) (end 64.5 56) (width 0.3) (layer B.Cu) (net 6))
 (segment (start 62.42 67) (end 62.42 63.08) (width 0.5) (layer B.Cu) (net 21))
 (segment (start 62.42 63.08) (end 64.5 61) (width 0.5) (layer B.Cu) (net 21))
 (segment (start 69.5 31.5) (end 69.5 43) (width 0.5) (layer B.Cu) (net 13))
 (segment (start 74 47.5) (end 69.5 43) (width 0.5) (layer B.Cu) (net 13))
 (segment (start 74 47.5) (end 74 49) (width 0.5) (layer B.Cu) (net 13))
 (segment (start 77.66 67) (end 77.66 57.66) (width 0.5) (layer B.Cu) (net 22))
 (segment (start 77.66 57.66) (end 74 54) (width 0.5) (layer B.Cu) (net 22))
 (segment (start 68.5 27.5) (end 68.5 53.5) (width 0.3) (layer B.Cu) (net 5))
 (segment (start 68.5 53.5) (end 70.5 55.5) (width 0.3) (layer B.Cu) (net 5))
 (segment (start 70.5 55.5) (end 70.5 56) (width 0.3) (layer B.Cu) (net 5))
 (segment (start 72.58 67) (end 72.58 63.08) (width 0.5) (layer B.Cu) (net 23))
 (segment (start 72.58 63.08) (end 70.5 61) (width 0.5) (layer B.Cu) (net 23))
 (segment (start 65.5 31.5) (end 65.5 43) (width 0.5) (layer B.Cu) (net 14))
 (segment (start 61.5 47) (end 61.5 49) (width 0.5) (layer B.Cu) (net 14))
 (segment (start 61.5 47) (end 65.5 43) (width 0.5) (layer B.Cu) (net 14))
 (segment (start 57.34 67) (end 57.34 58.16) (width 0.5) (layer B.Cu) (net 24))
 (segment (start 57.34 58.16) (end 61.5 54) (width 0.5) (layer B.Cu) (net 24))
 (segment (start 55.5 31.5) (end 54 31.5) (width 0.5) (layer B.Cu) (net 20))
 (segment (start 48.5 45.5) (end 48.5 47) (width 0.5) (layer B.Cu) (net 20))
 (segment (start 52 42) (end 48.5 45.5) (width 0.5) (layer B.Cu) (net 20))
 (segment (start 52 33.5) (end 52 42) (width 0.5) (layer B.Cu) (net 20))
 (segment (start 54 31.5) (end 52 33.5) (width 0.5) (layer B.Cu) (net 20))
 (segment (start 64.5 27.5) (end 64.5 28.5) (width 0.5) (layer B.Cu) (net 7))
 (segment (start 50.5 40) (end 48.5 42) (width 0.5) (layer B.Cu) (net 7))
 (segment (start 50.5 32) (end 50.5 40) (width 0.5) (layer B.Cu) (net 7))
 (segment (start 52.5 30) (end 50.5 32) (width 0.5) (layer B.Cu) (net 7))
 (segment (start 63 30) (end 52.5 30) (width 0.5) (layer B.Cu) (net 7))
 (segment (start 64.5 28.5) (end 63 30) (width 0.5) (layer B.Cu) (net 7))
 (segment (start 79.5 31.5) (end 79.5 33.5) (width 0.5) (layer B.Cu) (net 8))
 (segment (start 88 45.5) (end 88 47) (width 0.5) (layer B.Cu) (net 8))
 (segment (start 82.5 40) (end 88 45.5) (width 0.5) (layer B.Cu) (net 8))
 (segment (start 82.5 36.5) (end 82.5 40) (width 0.5) (layer B.Cu) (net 8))
 (segment (start 79.5 33.5) (end 82.5 36.5) (width 0.5) (layer B.Cu) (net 8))
 (segment (start 79.5 31.5) (end 79.5 32) (width 0.5) (layer B.Cu) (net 8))
 (segment (start 70.5 27.5) (end 70.5 29) (width 0.5) (layer B.Cu) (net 4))
 (segment (start 87.5 42.5) (end 95.5 42.5) (width 0.5) (layer B.Cu) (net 4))
 (segment (start 84 39) (end 87.5 42.5) (width 0.5) (layer B.Cu) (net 4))
 (segment (start 84 33) (end 84 39) (width 0.5) (layer B.Cu) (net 4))
 (segment (start 81 30) (end 84 33) (width 0.5) (layer B.Cu) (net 4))
 (segment (start 71.5 30) (end 81 30) (width 0.5) (layer B.Cu) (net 4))
 (segment (start 70.5 29) (end 71.5 30) (width 0.5) (layer B.Cu) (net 4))
 (segment (start 76.5 27.5) (end 76.5 28) (width 0.5) (layer B.Cu) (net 2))
 (segment (start 76.5 28) (end 77.5 29) (width 0.5) (layer B.Cu) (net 2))
 (segment (start 77.5 29) (end 82 29) (width 0.5) (layer B.Cu) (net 2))
 (segment (start 82 29) (end 85.5 32.5) (width 0.5) (layer B.Cu) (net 2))
 (segment (start 85.5 32.5) (end 85.5 38.5) (width 0.5) (layer B.Cu) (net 2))
 (segment (start 85.5 38.5) (end 88 41) (width 0.5) (layer B.Cu) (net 2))
 (segment (start 88 41) (end 92 41) (width 0.5) (layer B.Cu) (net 2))
 (segment (start 92 41) (end 94 39) (width 0.5) (layer B.Cu) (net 2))
 (segment (start 94 39) (end 94 37) (width 0.5) (layer B.Cu) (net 2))
 (segment (start 94 37) (end 95.5 35.5) (width 0.5) (layer B.Cu) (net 2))
 (segment (start 77.5 31.5) (end 77.5 39) (width 1) (layer B.Cu) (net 9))
 (segment (start 99.04 65.04) (end 98.29 67) (width 1) (layer B.Cu) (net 9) (status 20))
 (segment (start 85 51) (end 99.04 65.04) (width 1) (layer B.Cu) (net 9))
 (segment (start 85 46.5) (end 85 51) (width 1) (layer B.Cu) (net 9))
 (segment (start 77.5 39) (end 85 46.5) (width 1) (layer B.Cu) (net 9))
 (segment (start 75.5 31.5) (end 75.5 40) (width 1) (layer B.Cu) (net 10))
 (segment (start 93.96 63.46) (end 93.21 67) (width 1) (layer B.Cu) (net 10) (status 20))
 (segment (start 83 52.5) (end 93.96 63.46) (width 1) (layer B.Cu) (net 10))
 (segment (start 83 47.5) (end 83 52.5) (width 1) (layer B.Cu) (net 10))
 (segment (start 75.5 40) (end 83 47.5) (width 1) (layer B.Cu) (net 10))
 (segment (start 73.5 31.5) (end 73.5 41) (width 1) (layer B.Cu) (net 11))
 (segment (start 88.04 60.54) (end 88.04 67) (width 1) (layer B.Cu) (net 11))
 (segment (start 81 53.5) (end 88.04 60.54) (width 1) (layer B.Cu) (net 11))
 (segment (start 81 48.5) (end 81 53.5) (width 1) (layer B.Cu) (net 11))
 (segment (start 73.5 41) (end 81 48.5) (width 1) (layer B.Cu) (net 11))
 (segment (start 71.5 31.5) (end 71.5 42) (width 1) (layer B.Cu) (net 12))
 (segment (start 82.96 58.96) (end 82.96 67) (width 1) (layer B.Cu) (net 12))
 (segment (start 79 55) (end 82.96 58.96) (width 1) (layer B.Cu) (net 12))
 (segment (start 79 49.5) (end 79 55) (width 1) (layer B.Cu) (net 12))
 (segment (start 71.5 42) (end 79 49.5) (width 1) (layer B.Cu) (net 12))
 (segment (start 63.5 31.5) (end 63.5 42) (width 1) (layer B.Cu) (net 15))
 (segment (start 52.04 59.96) (end 52.04 67) (width 1) (layer B.Cu) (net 15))
 (segment (start 57 55) (end 52.04 59.96) (width 1) (layer B.Cu) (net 15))
 (segment (start 57 48.5) (end 57 55) (width 1) (layer B.Cu) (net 15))
 (segment (start 63.5 42) (end 57 48.5) (width 1) (layer B.Cu) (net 15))
 (segment (start 61.5 31.5) (end 61.5 41) (width 1) (layer B.Cu) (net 16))
 (segment (start 46.96 62.04) (end 46.96 67) (width 1) (layer B.Cu) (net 16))
 (segment (start 55 54) (end 46.96 62.04) (width 1) (layer B.Cu) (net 16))
 (segment (start 55 47.5) (end 55 54) (width 1) (layer B.Cu) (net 16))
 (segment (start 61.5 41) (end 55 47.5) (width 1) (layer B.Cu) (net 16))
 (segment (start 59.5 31.5) (end 59.5 40) (width 1) (layer B.Cu) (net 18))
 (segment (start 40.54 65.46) (end 41.79 67) (width 1) (layer B.Cu) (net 18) (status 20))
 (segment (start 53 53) (end 40.54 65.46) (width 1) (layer B.Cu) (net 18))
 (segment (start 53 46.5) (end 53 53) (width 1) (layer B.Cu) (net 18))
 (segment (start 59.5 40) (end 53 46.5) (width 1) (layer B.Cu) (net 18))
 (segment (start 57.5 31.5) (end 57.5 39.5) (width 1) (layer B.Cu) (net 19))
 (segment (start 35.46 63.54) (end 36.71 67) (width 1) (layer B.Cu) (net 19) (status 20))
 (segment (start 37.5 61.5) (end 35.46 63.54) (width 1) (layer B.Cu) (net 19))
 (segment (start 41 61.5) (end 37.5 61.5) (width 1) (layer B.Cu) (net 19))
 (segment (start 51 51.5) (end 41 61.5) (width 1) (layer B.Cu) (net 19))
 (segment (start 51 46) (end 51 51.5) (width 1) (layer B.Cu) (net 19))
 (segment (start 57.5 39.5) (end 51 46) (width 1) (layer B.Cu) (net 19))
 (segment (start 21 29.5) (end 19.5 29.5) (width 1.1) (layer B.Cu) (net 25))
 (segment (start 18 31) (end 18 60.5) (width 1.1) (layer B.Cu) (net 25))
 (segment (start 19.5 29.5) (end 18 31) (width 1.1) (layer B.Cu) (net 25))
 (segment (start 18 60.5) (end 18.5 61) (width 1.1) (layer B.Cu) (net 25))
 (segment (start 21 34.58) (end 21 39.9981) (width 0.5) (layer B.Cu) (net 26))
 (segment (start 21 39.9981) (end 20.9981 40) (width 0.5) (layer B.Cu) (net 26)))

